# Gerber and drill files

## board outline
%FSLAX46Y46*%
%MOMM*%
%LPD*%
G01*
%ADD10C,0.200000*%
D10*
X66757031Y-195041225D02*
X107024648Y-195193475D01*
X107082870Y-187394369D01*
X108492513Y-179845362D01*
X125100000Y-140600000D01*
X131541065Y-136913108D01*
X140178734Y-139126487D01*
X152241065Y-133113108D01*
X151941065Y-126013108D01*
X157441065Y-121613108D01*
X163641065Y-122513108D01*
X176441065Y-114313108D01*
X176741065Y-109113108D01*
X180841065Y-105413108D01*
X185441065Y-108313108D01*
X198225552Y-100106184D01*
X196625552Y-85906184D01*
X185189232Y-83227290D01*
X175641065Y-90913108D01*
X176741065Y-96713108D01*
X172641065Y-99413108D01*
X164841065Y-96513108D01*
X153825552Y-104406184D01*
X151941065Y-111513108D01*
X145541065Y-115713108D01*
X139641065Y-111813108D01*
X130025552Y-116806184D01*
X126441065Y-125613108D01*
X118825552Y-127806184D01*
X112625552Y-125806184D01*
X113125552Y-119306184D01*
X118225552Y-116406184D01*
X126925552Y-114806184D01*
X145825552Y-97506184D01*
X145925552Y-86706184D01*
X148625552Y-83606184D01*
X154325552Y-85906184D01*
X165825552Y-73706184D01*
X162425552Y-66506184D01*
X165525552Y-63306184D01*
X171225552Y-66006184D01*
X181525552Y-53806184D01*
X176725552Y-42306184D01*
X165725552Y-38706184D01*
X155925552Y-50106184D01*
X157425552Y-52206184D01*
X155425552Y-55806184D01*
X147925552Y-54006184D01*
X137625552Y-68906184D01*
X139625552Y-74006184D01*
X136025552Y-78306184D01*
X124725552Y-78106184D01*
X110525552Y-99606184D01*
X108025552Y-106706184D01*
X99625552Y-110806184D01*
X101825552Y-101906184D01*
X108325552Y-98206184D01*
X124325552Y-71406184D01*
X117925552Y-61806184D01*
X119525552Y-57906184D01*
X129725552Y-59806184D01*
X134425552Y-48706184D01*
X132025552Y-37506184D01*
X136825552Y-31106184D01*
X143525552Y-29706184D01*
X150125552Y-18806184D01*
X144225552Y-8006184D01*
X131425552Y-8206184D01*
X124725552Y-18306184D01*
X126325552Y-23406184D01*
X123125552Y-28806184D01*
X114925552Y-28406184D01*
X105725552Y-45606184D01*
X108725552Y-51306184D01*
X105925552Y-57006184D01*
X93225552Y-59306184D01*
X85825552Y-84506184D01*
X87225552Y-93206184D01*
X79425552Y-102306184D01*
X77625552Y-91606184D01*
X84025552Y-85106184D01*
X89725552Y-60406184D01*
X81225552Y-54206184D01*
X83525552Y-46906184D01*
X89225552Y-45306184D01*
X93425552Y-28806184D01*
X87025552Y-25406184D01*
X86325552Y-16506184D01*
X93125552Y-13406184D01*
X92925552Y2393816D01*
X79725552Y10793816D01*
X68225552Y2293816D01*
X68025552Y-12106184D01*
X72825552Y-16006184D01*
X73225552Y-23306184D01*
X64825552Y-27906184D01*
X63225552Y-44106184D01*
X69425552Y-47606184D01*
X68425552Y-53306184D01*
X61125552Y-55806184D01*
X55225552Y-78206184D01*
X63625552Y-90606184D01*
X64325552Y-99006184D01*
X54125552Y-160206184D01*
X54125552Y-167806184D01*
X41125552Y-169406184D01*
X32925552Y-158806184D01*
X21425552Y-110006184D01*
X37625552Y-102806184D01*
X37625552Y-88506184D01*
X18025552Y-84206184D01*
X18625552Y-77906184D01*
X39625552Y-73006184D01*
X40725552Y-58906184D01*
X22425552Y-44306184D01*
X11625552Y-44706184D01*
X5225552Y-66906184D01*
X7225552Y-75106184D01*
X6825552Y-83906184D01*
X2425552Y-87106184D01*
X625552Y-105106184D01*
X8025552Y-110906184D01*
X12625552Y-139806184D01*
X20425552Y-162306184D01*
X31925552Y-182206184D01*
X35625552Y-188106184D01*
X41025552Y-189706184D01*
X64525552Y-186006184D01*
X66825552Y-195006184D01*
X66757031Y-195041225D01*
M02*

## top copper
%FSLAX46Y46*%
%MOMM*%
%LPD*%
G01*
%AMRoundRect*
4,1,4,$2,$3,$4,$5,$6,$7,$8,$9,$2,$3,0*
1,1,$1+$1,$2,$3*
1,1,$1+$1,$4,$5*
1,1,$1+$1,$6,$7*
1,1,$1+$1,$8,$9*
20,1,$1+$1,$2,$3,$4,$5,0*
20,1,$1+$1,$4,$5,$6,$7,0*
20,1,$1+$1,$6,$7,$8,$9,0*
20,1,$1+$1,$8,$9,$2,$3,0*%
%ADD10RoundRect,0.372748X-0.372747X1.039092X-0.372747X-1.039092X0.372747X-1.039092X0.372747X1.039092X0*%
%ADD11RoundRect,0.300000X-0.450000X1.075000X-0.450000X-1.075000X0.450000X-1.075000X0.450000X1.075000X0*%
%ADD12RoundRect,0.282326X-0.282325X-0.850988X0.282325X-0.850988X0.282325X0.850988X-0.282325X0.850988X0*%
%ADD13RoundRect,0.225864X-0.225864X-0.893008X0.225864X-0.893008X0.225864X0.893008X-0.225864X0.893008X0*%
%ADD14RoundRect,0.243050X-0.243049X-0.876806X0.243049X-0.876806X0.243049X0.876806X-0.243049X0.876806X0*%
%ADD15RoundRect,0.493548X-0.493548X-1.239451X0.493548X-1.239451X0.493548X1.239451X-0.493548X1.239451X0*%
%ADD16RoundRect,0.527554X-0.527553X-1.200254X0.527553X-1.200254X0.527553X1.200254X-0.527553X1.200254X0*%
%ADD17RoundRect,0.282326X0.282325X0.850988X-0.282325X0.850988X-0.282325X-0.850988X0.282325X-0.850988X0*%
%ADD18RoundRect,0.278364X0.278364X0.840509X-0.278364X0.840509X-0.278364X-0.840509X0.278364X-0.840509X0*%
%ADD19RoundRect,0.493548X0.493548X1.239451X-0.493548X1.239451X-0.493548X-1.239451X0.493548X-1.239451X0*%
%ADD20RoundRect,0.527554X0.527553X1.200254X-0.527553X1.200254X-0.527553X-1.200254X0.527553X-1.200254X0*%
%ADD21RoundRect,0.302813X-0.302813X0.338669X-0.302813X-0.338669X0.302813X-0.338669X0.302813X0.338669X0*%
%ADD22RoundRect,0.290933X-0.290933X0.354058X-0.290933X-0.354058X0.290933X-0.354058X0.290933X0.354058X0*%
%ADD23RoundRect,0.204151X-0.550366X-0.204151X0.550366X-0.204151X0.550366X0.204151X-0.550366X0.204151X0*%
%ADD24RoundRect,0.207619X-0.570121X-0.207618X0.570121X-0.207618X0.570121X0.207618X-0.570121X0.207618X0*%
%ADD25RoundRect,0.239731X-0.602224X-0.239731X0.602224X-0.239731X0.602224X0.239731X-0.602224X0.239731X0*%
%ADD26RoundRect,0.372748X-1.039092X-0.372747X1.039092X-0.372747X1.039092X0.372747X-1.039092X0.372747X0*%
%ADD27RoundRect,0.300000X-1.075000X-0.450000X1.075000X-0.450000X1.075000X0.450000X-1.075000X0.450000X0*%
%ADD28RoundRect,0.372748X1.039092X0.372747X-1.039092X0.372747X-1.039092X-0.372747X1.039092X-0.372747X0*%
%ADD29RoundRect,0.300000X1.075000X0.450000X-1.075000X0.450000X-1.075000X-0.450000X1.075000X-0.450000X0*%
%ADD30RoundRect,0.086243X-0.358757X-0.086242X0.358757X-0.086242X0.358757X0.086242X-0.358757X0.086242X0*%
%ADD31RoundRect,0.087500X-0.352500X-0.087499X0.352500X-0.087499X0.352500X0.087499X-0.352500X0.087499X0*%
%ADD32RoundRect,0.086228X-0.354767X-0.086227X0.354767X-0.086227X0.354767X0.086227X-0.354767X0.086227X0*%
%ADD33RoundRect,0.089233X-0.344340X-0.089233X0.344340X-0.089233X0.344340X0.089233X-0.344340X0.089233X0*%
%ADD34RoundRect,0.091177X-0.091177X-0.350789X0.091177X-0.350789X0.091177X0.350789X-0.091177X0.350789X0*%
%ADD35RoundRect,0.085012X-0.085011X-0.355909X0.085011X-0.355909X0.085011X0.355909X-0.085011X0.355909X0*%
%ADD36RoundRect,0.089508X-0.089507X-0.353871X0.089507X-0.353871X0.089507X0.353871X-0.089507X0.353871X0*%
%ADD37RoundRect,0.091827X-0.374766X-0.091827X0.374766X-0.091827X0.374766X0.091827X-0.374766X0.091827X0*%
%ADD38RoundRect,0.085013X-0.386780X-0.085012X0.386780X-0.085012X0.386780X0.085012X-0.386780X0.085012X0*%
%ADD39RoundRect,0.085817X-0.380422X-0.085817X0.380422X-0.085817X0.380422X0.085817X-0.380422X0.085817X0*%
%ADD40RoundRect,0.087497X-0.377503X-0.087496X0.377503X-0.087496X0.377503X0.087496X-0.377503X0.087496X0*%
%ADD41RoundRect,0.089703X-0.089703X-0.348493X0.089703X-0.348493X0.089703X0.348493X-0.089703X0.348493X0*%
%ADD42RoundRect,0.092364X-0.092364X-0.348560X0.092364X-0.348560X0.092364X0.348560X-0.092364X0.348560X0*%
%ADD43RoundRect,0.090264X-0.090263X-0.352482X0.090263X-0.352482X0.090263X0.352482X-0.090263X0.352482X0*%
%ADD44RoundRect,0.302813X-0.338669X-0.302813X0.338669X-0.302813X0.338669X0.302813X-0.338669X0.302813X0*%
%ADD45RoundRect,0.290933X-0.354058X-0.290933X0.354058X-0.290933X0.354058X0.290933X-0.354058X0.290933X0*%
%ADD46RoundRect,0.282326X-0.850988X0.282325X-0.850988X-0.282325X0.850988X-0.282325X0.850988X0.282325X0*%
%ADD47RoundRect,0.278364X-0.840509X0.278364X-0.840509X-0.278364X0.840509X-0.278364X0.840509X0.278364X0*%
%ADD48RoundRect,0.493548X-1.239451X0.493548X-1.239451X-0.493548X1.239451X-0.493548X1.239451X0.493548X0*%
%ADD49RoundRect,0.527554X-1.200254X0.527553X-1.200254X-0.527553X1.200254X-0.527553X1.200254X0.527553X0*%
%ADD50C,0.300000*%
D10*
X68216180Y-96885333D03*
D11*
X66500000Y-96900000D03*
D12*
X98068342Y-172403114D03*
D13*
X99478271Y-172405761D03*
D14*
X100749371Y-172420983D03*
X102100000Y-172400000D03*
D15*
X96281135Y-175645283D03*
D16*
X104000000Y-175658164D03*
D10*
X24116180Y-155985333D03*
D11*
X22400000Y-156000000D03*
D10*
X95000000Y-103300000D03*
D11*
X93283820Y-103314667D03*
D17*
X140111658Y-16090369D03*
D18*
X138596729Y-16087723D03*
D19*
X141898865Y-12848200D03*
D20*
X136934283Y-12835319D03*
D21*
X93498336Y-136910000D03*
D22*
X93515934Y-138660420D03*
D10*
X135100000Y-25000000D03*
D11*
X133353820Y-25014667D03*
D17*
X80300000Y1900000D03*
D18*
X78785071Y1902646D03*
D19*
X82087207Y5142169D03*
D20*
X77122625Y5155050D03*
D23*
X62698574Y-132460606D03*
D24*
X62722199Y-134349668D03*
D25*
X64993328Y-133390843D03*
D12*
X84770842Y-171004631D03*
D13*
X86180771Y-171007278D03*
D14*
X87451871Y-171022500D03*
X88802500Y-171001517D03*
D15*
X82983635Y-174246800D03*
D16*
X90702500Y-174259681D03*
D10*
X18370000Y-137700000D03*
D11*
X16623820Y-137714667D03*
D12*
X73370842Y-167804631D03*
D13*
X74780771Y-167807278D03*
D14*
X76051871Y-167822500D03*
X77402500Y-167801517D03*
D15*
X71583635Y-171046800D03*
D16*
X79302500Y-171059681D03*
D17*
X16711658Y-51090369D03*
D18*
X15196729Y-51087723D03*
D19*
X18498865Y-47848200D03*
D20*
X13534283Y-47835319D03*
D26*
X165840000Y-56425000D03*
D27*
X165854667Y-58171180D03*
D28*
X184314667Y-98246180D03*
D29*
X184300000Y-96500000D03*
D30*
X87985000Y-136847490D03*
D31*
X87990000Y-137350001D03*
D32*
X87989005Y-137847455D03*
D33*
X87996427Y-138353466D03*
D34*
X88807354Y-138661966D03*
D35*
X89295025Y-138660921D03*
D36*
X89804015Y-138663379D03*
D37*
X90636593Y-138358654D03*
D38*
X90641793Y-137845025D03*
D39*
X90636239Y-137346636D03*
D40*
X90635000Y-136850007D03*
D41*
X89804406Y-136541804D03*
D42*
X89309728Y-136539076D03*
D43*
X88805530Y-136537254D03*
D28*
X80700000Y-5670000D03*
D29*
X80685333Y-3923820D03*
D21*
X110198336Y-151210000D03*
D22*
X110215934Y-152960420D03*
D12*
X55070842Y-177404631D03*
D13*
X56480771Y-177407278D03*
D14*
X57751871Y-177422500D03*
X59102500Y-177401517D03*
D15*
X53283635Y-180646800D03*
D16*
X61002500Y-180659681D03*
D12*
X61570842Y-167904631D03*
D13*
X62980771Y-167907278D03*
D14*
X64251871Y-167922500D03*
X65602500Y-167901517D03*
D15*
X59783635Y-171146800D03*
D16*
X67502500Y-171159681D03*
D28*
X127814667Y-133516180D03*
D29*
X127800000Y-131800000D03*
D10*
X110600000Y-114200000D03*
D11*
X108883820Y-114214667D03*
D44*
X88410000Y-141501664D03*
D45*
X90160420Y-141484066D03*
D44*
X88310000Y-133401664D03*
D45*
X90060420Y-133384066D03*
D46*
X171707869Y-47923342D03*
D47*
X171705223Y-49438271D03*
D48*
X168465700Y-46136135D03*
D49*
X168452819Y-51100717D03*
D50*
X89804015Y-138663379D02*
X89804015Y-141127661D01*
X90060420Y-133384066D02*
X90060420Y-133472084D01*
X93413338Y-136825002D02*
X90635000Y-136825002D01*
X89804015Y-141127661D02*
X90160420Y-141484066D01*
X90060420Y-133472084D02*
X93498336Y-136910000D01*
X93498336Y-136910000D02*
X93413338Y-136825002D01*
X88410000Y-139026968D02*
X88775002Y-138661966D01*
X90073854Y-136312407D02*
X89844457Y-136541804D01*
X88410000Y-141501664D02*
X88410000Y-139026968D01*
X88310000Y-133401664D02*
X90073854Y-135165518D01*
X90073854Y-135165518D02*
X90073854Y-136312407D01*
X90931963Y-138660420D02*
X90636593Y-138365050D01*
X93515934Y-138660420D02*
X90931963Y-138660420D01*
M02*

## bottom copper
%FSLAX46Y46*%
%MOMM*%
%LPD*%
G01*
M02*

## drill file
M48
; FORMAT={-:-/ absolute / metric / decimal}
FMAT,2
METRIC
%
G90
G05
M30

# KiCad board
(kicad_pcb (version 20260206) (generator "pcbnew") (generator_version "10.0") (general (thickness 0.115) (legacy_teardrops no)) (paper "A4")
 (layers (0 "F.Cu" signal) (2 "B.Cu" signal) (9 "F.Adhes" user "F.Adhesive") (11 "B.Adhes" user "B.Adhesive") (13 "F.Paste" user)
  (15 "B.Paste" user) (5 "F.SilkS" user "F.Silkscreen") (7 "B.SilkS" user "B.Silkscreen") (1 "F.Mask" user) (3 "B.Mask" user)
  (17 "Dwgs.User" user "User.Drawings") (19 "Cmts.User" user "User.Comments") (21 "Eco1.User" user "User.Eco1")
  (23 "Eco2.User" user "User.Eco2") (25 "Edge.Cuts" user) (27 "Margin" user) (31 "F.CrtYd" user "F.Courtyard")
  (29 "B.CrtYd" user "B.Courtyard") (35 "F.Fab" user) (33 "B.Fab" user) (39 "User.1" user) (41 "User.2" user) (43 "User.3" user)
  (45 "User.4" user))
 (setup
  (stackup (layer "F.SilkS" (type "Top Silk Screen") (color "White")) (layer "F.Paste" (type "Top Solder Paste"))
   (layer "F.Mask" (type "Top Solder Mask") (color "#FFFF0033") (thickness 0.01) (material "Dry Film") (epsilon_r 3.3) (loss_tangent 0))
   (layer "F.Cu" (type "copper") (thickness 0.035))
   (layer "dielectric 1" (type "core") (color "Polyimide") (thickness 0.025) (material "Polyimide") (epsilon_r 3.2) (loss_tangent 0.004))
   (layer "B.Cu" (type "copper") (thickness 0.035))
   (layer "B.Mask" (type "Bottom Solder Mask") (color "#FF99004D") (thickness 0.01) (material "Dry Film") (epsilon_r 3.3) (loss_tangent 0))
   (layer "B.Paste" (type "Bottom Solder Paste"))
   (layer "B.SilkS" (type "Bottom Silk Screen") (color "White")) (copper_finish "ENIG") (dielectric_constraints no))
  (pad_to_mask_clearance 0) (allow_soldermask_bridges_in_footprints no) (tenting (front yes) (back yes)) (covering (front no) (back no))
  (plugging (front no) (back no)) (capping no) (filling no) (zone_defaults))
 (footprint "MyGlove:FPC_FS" (layer "F.Cu") (at 67.37618 96.885333)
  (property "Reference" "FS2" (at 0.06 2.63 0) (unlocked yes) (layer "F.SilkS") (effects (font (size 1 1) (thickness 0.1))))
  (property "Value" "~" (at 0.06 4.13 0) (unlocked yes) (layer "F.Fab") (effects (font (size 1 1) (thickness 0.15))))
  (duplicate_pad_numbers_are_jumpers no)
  (pad "" smd roundrect (at -0.75 0.01 270) (size 2 1) (layers "F.Mask" "F.Paste") (roundrect_rratio 0.2)
   (teardrops (best_length_ratio 0.5) (max_length 1) (best_width_ratio 1) (max_width 2) (curved_edges yes) (filter_ratio 0.9) (enabled yes)
    (allow_two_segments yes) (prefer_zone_connections yes)))
  (pad "" smd roundrect (at 0.75 0.01 270) (size 2 1) (layers "F.Mask" "F.Paste") (roundrect_rratio 0.2)
   (teardrops (best_length_ratio 0.5) (max_length 1) (best_width_ratio 1) (max_width 2) (curved_edges yes) (filter_ratio 0.9) (enabled yes)
    (allow_two_segments yes) (prefer_zone_connections yes)))
  (pad "1" smd roundrect (at 0.84 0 270) (size 2.82368 1.49099) (layers "F.Cu") (roundrect_rratio 0.25) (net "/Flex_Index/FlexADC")
   (teardrops (best_length_ratio 0.5) (max_length 1) (best_width_ratio 1) (max_width 2) (curved_edges yes) (filter_ratio 0.9) (enabled yes)
    (allow_two_segments yes) (prefer_zone_connections yes))
   (padstack (mode custom) (layer "B.Cu" (shape roundrect) (size 2.177876 1.183907) (roundrect_rratio 0.25) (zone_connect -1))))
  (pad "2" smd roundrect (at -0.87618 0.014667 270) (size 2.75 1.5) (layers "F.Cu") (roundrect_rratio 0.2) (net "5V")
   (teardrops (best_length_ratio 0.5) (max_length 1) (best_width_ratio 1) (max_width 2) (curved_edges yes) (filter_ratio 0.9) (enabled yes)
    (allow_two_segments yes) (prefer_zone_connections yes))))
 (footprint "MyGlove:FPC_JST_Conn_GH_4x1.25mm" (layer "F.Cu") (at 95.28 177.970983)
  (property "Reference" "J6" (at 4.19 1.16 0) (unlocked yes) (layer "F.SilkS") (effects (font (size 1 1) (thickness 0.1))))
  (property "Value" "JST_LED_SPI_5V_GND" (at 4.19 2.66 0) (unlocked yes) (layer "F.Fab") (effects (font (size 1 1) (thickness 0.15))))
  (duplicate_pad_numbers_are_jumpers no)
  (pad "" smd roundrect (at 1.065 -2.46) (size 1 2.7) (layers "F.Mask" "F.Paste") (roundrect_rratio 0.25))
  (pad "" smd roundrect (at 2.915 -5.66) (size 0.6 1.7) (layers "F.Mask" "F.Paste") (roundrect_rratio 0.25))
  (pad "" smd roundrect (at 4.165 -5.66) (size 0.6 1.7) (layers "F.Mask" "F.Paste") (roundrect_rratio 0.25))
  (pad "" smd roundrect (at 5.48 -5.61) (size 0.6 1.7) (layers "F.Mask" "F.Paste") (roundrect_rratio 0.25))
  (pad "" smd roundrect (at 6.74 -5.650983) (size 0.6 1.7) (layers "F.Mask" "F.Paste") (roundrect_rratio 0.25))
  (pad "" smd roundrect (at 8.56 -2.46) (size 1 2.7) (layers "F.Mask" "F.Paste") (roundrect_rratio 0.25))
  (pad "1" smd roundrect (at 2.788342 -5.567869) (size 1.129302 2.266628) (layers "F.Cu") (roundrect_rratio 0.25) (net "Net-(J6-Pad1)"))
  (pad "2" smd roundrect (at 4.198271 -5.565222) (size 0.903457 2.237745) (layers "F.Cu") (roundrect_rratio 0.25) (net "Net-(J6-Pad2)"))
  (pad "3" smd roundrect (at 5.469371 -5.55) (size 0.972199 2.239712) (layers "F.Cu") (roundrect_rratio 0.25) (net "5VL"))
  (pad "4" smd roundrect (at 6.82 -5.570983) (size 0.972199 2.239712) (layers "F.Cu") (roundrect_rratio 0.25) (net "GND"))
  (pad "MP" smd roundrect (at 1.001135 -2.3257) (size 1.974193 3.465998) (layers "F.Cu") (roundrect_rratio 0.25))
  (pad "MP" smd roundrect (at 8.72 -2.312819) (size 2.110214 3.455616) (layers "F.Cu") (roundrect_rratio 0.25)))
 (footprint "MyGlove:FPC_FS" (layer "F.Cu") (at 23.27618 155.985333)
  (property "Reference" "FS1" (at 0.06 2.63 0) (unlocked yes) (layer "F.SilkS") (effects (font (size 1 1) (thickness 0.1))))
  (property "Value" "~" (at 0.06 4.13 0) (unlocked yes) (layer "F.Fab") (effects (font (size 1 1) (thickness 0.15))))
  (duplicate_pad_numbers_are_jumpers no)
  (pad "" smd roundrect (at -0.75 0.01 270) (size 2 1) (layers "F.Mask" "F.Paste") (roundrect_rratio 0.2)
   (teardrops (best_length_ratio 0.5) (max_length 1) (best_width_ratio 1) (max_width 2) (curved_edges yes) (filter_ratio 0.9) (enabled yes)
    (allow_two_segments yes) (prefer_zone_connections yes)))
  (pad "" smd roundrect (at 0.75 0.01 270) (size 2 1) (layers "F.Mask" "F.Paste") (roundrect_rratio 0.2)
   (teardrops (best_length_ratio 0.5) (max_length 1) (best_width_ratio 1) (max_width 2) (curved_edges yes) (filter_ratio 0.9) (enabled yes)
    (allow_two_segments yes) (prefer_zone_connections yes)))
  (pad "1" smd roundrect (at 0.84 0 270) (size 2.82368 1.49099) (layers "F.Cu") (roundrect_rratio 0.25) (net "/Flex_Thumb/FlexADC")
   (teardrops (best_length_ratio 0.5) (max_length 1) (best_width_ratio 1) (max_width 2) (curved_edges yes) (filter_ratio 0.9) (enabled yes)
    (allow_two_segments yes) (prefer_zone_connections yes))
   (padstack (mode custom) (layer "B.Cu" (shape roundrect) (size 2.177876 1.183907) (roundrect_rratio 0.25) (zone_connect -1))))
  (pad "2" smd roundrect (at -0.87618 0.014667 270) (size 2.75 1.5) (layers "F.Cu") (roundrect_rratio 0.2) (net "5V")
   (teardrops (best_length_ratio 0.5) (max_length 1) (best_width_ratio 1) (max_width 2) (curved_edges yes) (filter_ratio 0.9) (enabled yes)
    (allow_two_segments yes) (prefer_zone_connections yes))))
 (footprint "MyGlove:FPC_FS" (layer "F.Cu") (at 94.16 103.3)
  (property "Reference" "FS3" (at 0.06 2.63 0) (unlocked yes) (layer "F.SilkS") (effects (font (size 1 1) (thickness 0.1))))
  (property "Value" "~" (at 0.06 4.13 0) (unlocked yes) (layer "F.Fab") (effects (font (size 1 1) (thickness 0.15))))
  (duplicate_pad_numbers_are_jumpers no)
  (pad "" smd roundrect (at -0.75 0.01 270) (size 2 1) (layers "F.Mask" "F.Paste") (roundrect_rratio 0.2)
   (teardrops (best_length_ratio 0.5) (max_length 1) (best_width_ratio 1) (max_width 2) (curved_edges yes) (filter_ratio 0.9) (enabled yes)
    (allow_two_segments yes) (prefer_zone_connections yes)))
  (pad "" smd roundrect (at 0.75 0.01 270) (size 2 1) (layers "F.Mask" "F.Paste") (roundrect_rratio 0.2)
   (teardrops (best_length_ratio 0.5) (max_length 1) (best_width_ratio 1) (max_width 2) (curved_edges yes) (filter_ratio 0.9) (enabled yes)
    (allow_two_segments yes) (prefer_zone_connections yes)))
  (pad "1" smd roundrect (at 0.84 0 270) (size 2.82368 1.49099) (layers "F.Cu") (roundrect_rratio 0.25) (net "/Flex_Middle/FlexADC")
   (teardrops (best_length_ratio 0.5) (max_length 1) (best_width_ratio 1) (max_width 2) (curved_edges yes) (filter_ratio 0.9) (enabled yes)
    (allow_two_segments yes) (prefer_zone_connections yes))
   (padstack (mode custom) (layer "B.Cu" (shape roundrect) (size 2.177876 1.183907) (roundrect_rratio 0.25) (zone_connect -1))))
  (pad "2" smd roundrect (at -0.87618 0.014667 270) (size 2.75 1.5) (layers "F.Cu") (roundrect_rratio 0.2) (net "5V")
   (teardrops (best_length_ratio 0.5) (max_length 1) (best_width_ratio 1) (max_width 2) (curved_edges yes) (filter_ratio 0.9) (enabled yes)
    (allow_two_segments yes) (prefer_zone_connections yes))))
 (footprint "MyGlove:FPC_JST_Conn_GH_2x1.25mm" (layer "F.Cu") (at 142.9 10.5225 180)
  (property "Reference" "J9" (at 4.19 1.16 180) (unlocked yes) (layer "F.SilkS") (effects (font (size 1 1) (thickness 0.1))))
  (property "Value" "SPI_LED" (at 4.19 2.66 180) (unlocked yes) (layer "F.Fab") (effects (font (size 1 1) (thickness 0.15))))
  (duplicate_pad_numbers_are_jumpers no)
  (pad "" smd roundrect (at 1.065 -2.46 180) (size 1 2.7) (layers "F.Mask" "F.Paste") (roundrect_rratio 0.25))
  (pad "" smd roundrect (at 2.915 -5.66 180) (size 0.6 1.7) (layers "F.Mask" "F.Paste") (roundrect_rratio 0.25))
  (pad "" smd roundrect (at 4.165 -5.66 180) (size 0.6 1.7) (layers "F.Mask" "F.Paste") (roundrect_rratio 0.25))
  (pad "" smd roundrect (at 6.015 -2.46 180) (size 1 2.7) (layers "F.Mask" "F.Paste") (roundrect_rratio 0.25))
  (pad "1" smd roundrect (at 2.788342 -5.567869 180) (size 1.129302 2.266628) (layers "F.Cu") (roundrect_rratio 0.25) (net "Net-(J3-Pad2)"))
  (pad "2" smd roundrect (at 4.303271 -5.565223 180) (size 1.113457 2.237746) (layers "F.Cu") (roundrect_rratio 0.25) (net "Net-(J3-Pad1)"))
  (pad "MP" smd roundrect (at 1.001135 -2.3257 180) (size 1.974193 3.465998) (layers "F.Cu") (roundrect_rratio 0.25))
  (pad "MP" smd roundrect (at 5.965717 -2.312819 180) (size 2.110214 3.455616) (layers "F.Cu") (roundrect_rratio 0.25)))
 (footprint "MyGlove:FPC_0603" (layer "F.Cu") (at 93.5 137.8 -90)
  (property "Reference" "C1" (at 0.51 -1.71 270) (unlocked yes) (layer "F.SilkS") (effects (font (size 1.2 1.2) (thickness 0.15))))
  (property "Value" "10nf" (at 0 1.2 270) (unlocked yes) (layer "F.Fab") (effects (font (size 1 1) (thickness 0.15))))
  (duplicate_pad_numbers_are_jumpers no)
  (pad "" smd roundrect (at -0.87 0.005971 270) (size 1.00047 0.948058) (layers "F.Mask" "F.Paste") (roundrect_rratio 0.2))
  (pad "" smd roundrect (at 0.85 0 270) (size 1.054536 0.970792) (layers "F.Mask" "F.Paste") (roundrect_rratio 0.2))
  (pad "1" smd roundrect (at -0.89 0.001664 270) (size 1.282964 1.211252) (layers "F.Cu") (roundrect_rratio 0.25) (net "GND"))
  (pad "2" smd roundrect (at 0.86042 -0.015934 270) (size 1.289982 1.163733) (layers "F.Cu") (roundrect_rratio 0.25) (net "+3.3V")))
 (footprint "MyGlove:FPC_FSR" (layer "F.Cu") (at 134.23 25)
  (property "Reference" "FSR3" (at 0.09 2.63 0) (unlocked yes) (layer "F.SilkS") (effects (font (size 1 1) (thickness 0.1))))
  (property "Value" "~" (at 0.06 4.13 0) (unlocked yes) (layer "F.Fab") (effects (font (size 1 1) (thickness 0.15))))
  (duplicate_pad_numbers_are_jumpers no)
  (pad "" smd roundrect (at -0.75 0.01 270) (size 2 1) (layers "F.Mask" "F.Paste") (roundrect_rratio 0.2)
   (teardrops (best_length_ratio 0.5) (max_length 1) (best_width_ratio 1) (max_width 2) (curved_edges yes) (filter_ratio 0.9) (enabled yes)
    (allow_two_segments yes) (prefer_zone_connections yes)))
  (pad "" smd roundrect (at 0.78 0.01 270) (size 2 1) (layers "F.Mask" "F.Paste") (roundrect_rratio 0.2)
   (teardrops (best_length_ratio 0.5) (max_length 1) (best_width_ratio 1) (max_width 2) (curved_edges yes) (filter_ratio 0.9) (enabled yes)
    (allow_two_segments yes) (prefer_zone_connections yes)))
  (pad "1" smd roundrect (at 0.87 0 270) (size 2.82368 1.49099) (layers "F.Cu") (roundrect_rratio 0.25) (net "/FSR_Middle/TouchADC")
   (teardrops (best_length_ratio 0.5) (max_length 1) (best_width_ratio 1) (max_width 2) (curved_edges yes) (filter_ratio 0.9) (enabled yes)
    (allow_two_segments yes) (prefer_zone_connections yes))
   (padstack (mode custom) (layer "B.Cu" (shape roundrect) (size 2.177876 1.183907) (roundrect_rratio 0.25) (zone_connect -1))))
  (pad "2" smd roundrect (at -0.87618 0.014667 270) (size 2.75 1.5) (layers "F.Cu") (roundrect_rratio 0.2) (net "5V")
   (teardrops (best_length_ratio 0.5) (max_length 1) (best_width_ratio 1) (max_width 2) (curved_edges yes) (filter_ratio 0.9) (enabled yes)
    (allow_two_segments yes) (prefer_zone_connections yes))))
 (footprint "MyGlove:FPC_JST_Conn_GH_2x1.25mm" (layer "F.Cu") (at 83.088342 -7.467869 180)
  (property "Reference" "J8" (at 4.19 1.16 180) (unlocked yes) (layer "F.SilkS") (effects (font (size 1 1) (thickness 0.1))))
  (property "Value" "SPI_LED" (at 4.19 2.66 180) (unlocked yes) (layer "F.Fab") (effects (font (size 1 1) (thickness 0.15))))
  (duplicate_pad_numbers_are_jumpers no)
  (pad "" smd roundrect (at 1.065 -2.46 180) (size 1 2.7) (layers "F.Mask" "F.Paste") (roundrect_rratio 0.25))
  (pad "" smd roundrect (at 2.915 -5.66 180) (size 0.6 1.7) (layers "F.Mask" "F.Paste") (roundrect_rratio 0.25))
  (pad "" smd roundrect (at 4.165 -5.66 180) (size 0.6 1.7) (layers "F.Mask" "F.Paste") (roundrect_rratio 0.25))
  (pad "" smd roundrect (at 6.015 -2.46 180) (size 1 2.7) (layers "F.Mask" "F.Paste") (roundrect_rratio 0.25))
  (pad "1" smd roundrect (at 2.788342 -5.567869 180) (size 1.129302 2.266628) (layers "F.Cu") (roundrect_rratio 0.25) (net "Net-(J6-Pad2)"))
  (pad "2" smd roundrect (at 4.303271 -5.565223 180) (size 1.113457 2.237746) (layers "F.Cu") (roundrect_rratio 0.25) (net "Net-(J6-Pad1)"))
  (pad "MP" smd roundrect (at 1.001135 -2.3257 180) (size 1.974193 3.465998) (layers "F.Cu") (roundrect_rratio 0.25))
  (pad "MP" smd roundrect (at 5.965717 -2.312819 180) (size 2.110214 3.455616) (layers "F.Cu") (roundrect_rratio 0.25)))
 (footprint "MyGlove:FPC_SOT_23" (layer "F.Cu") (at 63.8425 133.37)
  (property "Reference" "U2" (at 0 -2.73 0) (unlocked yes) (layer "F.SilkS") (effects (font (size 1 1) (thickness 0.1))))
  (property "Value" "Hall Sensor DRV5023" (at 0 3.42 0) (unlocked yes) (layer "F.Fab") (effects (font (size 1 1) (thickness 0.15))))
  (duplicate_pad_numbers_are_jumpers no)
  (pad "" smd roundrect (at -1.1175 -0.92) (size 1.325 0.6) (layers "F.Mask" "F.Paste") (roundrect_rratio 0.25))
  (pad "" smd roundrect (at -1.1175 0.98) (size 1.325 0.6) (layers "F.Mask" "F.Paste") (roundrect_rratio 0.25))
  (pad "" smd roundrect (at 1.1575 0.03) (size 1.325 0.6) (layers "F.Mask" "F.Paste") (roundrect_rratio 0.25))
  (pad "1" smd roundrect (at -1.143926 -0.909394) (size 1.509034 0.816604) (layers "F.Cu") (roundrect_rratio 0.25) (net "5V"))
  (pad "2" smd roundrect (at -1.120301 0.979668) (size 1.555481 0.830475) (layers "F.Cu") (roundrect_rratio 0.25) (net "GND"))
  (pad "3" smd roundrect (at 1.150828 0.020843) (size 1.683911 0.958924) (layers "F.Cu") (roundrect_rratio 0.25)
   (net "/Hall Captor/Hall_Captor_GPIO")))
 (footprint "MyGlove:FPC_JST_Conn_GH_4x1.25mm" (layer "F.Cu") (at 81.9825 176.5725)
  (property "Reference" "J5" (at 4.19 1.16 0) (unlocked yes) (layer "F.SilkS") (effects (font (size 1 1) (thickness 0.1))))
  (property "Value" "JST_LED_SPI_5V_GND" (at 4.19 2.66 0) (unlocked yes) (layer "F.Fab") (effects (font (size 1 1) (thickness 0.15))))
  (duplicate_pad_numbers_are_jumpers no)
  (pad "" smd roundrect (at 1.065 -2.46) (size 1 2.7) (layers "F.Mask" "F.Paste") (roundrect_rratio 0.25))
  (pad "" smd roundrect (at 2.915 -5.66) (size 0.6 1.7) (layers "F.Mask" "F.Paste") (roundrect_rratio 0.25))
  (pad "" smd roundrect (at 4.165 -5.66) (size 0.6 1.7) (layers "F.Mask" "F.Paste") (roundrect_rratio 0.25))
  (pad "" smd roundrect (at 5.48 -5.61) (size 0.6 1.7) (layers "F.Mask" "F.Paste") (roundrect_rratio 0.25))
  (pad "" smd roundrect (at 6.74 -5.650983) (size 0.6 1.7) (layers "F.Mask" "F.Paste") (roundrect_rratio 0.25))
  (pad "" smd roundrect (at 8.56 -2.46) (size 1 2.7) (layers "F.Mask" "F.Paste") (roundrect_rratio 0.25))
  (pad "1" smd roundrect (at 2.788342 -5.567869) (size 1.129302 2.266628) (layers "F.Cu") (roundrect_rratio 0.25) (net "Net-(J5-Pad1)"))
  (pad "2" smd roundrect (at 4.198271 -5.565222) (size 0.903457 2.237745) (layers "F.Cu") (roundrect_rratio 0.25) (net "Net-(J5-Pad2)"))
  (pad "3" smd roundrect (at 5.469371 -5.55) (size 0.972199 2.239712) (layers "F.Cu") (roundrect_rratio 0.25) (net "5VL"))
  (pad "4" smd roundrect (at 6.82 -5.570983) (size 0.972199 2.239712) (layers "F.Cu") (roundrect_rratio 0.25) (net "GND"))
  (pad "MP" smd roundrect (at 1.001135 -2.3257) (size 1.974193 3.465998) (layers "F.Cu") (roundrect_rratio 0.25))
  (pad "MP" smd roundrect (at 8.72 -2.312819) (size 2.110214 3.455616) (layers "F.Cu") (roundrect_rratio 0.25)))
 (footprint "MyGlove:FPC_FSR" (layer "F.Cu") (at 17.5 137.7)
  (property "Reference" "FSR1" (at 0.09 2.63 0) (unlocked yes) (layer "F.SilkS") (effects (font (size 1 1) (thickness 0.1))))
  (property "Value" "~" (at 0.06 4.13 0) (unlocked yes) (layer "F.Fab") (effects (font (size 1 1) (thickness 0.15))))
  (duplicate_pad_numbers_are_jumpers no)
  (pad "" smd roundrect (at -0.75 0.01 270) (size 2 1) (layers "F.Mask" "F.Paste") (roundrect_rratio 0.2)
   (teardrops (best_length_ratio 0.5) (max_length 1) (best_width_ratio 1) (max_width 2) (curved_edges yes) (filter_ratio 0.9) (enabled yes)
    (allow_two_segments yes) (prefer_zone_connections yes)))
  (pad "" smd roundrect (at 0.78 0.01 270) (size 2 1) (layers "F.Mask" "F.Paste") (roundrect_rratio 0.2)
   (teardrops (best_length_ratio 0.5) (max_length 1) (best_width_ratio 1) (max_width 2) (curved_edges yes) (filter_ratio 0.9) (enabled yes)
    (allow_two_segments yes) (prefer_zone_connections yes)))
  (pad "1" smd roundrect (at 0.87 0 270) (size 2.82368 1.49099) (layers "F.Cu") (roundrect_rratio 0.25) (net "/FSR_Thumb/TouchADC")
   (teardrops (best_length_ratio 0.5) (max_length 1) (best_width_ratio 1) (max_width 2) (curved_edges yes) (filter_ratio 0.9) (enabled yes)
    (allow_two_segments yes) (prefer_zone_connections yes))
   (padstack (mode custom) (layer "B.Cu" (shape roundrect) (size 2.177876 1.183907) (roundrect_rratio 0.25) (zone_connect -1))))
  (pad "2" smd roundrect (at -0.87618 0.014667 270) (size 2.75 1.5) (layers "F.Cu") (roundrect_rratio 0.2) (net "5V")
   (teardrops (best_length_ratio 0.5) (max_length 1) (best_width_ratio 1) (max_width 2) (curved_edges yes) (filter_ratio 0.9) (enabled yes)
    (allow_two_segments yes) (prefer_zone_connections yes))))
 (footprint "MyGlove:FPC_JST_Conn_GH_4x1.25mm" (layer "F.Cu") (at 70.5825 173.3725)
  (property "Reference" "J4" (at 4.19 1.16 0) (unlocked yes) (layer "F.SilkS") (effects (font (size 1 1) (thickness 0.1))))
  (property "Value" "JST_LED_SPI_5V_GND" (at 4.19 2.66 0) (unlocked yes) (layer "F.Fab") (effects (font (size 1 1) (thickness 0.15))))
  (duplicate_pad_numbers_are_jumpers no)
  (pad "" smd roundrect (at 1.065 -2.46) (size 1 2.7) (layers "F.Mask" "F.Paste") (roundrect_rratio 0.25))
  (pad "" smd roundrect (at 2.915 -5.66) (size 0.6 1.7) (layers "F.Mask" "F.Paste") (roundrect_rratio 0.25))
  (pad "" smd roundrect (at 4.165 -5.66) (size 0.6 1.7) (layers "F.Mask" "F.Paste") (roundrect_rratio 0.25))
  (pad "" smd roundrect (at 5.48 -5.61) (size 0.6 1.7) (layers "F.Mask" "F.Paste") (roundrect_rratio 0.25))
  (pad "" smd roundrect (at 6.74 -5.650983) (size 0.6 1.7) (layers "F.Mask" "F.Paste") (roundrect_rratio 0.25))
  (pad "" smd roundrect (at 8.56 -2.46) (size 1 2.7) (layers "F.Mask" "F.Paste") (roundrect_rratio 0.25))
  (pad "1" smd roundrect (at 2.788342 -5.567869) (size 1.129302 2.266628) (layers "F.Cu") (roundrect_rratio 0.25)
   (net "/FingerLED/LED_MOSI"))
  (pad "2" smd roundrect (at 4.198271 -5.565222) (size 0.903457 2.237745) (layers "F.Cu") (roundrect_rratio 0.25) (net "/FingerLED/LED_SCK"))
  (pad "3" smd roundrect (at 5.469371 -5.55) (size 0.972199 2.239712) (layers "F.Cu") (roundrect_rratio 0.25) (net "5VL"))
  (pad "4" smd roundrect (at 6.82 -5.570983) (size 0.972199 2.239712) (layers "F.Cu") (roundrect_rratio 0.25) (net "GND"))
  (pad "MP" smd roundrect (at 1.001135 -2.3257) (size 1.974193 3.465998) (layers "F.Cu") (roundrect_rratio 0.25))
  (pad "MP" smd roundrect (at 8.72 -2.312819) (size 2.110214 3.455616) (layers "F.Cu") (roundrect_rratio 0.25)))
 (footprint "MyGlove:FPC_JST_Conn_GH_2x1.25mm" (layer "F.Cu") (at 19.5 45.5225 180)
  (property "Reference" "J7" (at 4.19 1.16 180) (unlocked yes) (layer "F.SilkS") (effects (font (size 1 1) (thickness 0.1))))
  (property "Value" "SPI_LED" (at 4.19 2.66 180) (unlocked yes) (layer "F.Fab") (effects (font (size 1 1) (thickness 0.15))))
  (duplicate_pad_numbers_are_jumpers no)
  (pad "" smd roundrect (at 1.065 -2.46 180) (size 1 2.7) (layers "F.Mask" "F.Paste") (roundrect_rratio 0.25))
  (pad "" smd roundrect (at 2.915 -5.66 180) (size 0.6 1.7) (layers "F.Mask" "F.Paste") (roundrect_rratio 0.25))
  (pad "" smd roundrect (at 4.165 -5.66 180) (size 0.6 1.7) (layers "F.Mask" "F.Paste") (roundrect_rratio 0.25))
  (pad "" smd roundrect (at 6.015 -2.46 180) (size 1 2.7) (layers "F.Mask" "F.Paste") (roundrect_rratio 0.25))
  (pad "1" smd roundrect (at 2.788342 -5.567869 180) (size 1.129302 2.266628) (layers "F.Cu") (roundrect_rratio 0.25) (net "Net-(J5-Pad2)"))
  (pad "2" smd roundrect (at 4.303271 -5.565223 180) (size 1.113457 2.237746) (layers "F.Cu") (roundrect_rratio 0.25) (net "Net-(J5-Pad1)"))
  (pad "MP" smd roundrect (at 1.001135 -2.3257 180) (size 1.974193 3.465998) (layers "F.Cu") (roundrect_rratio 0.25))
  (pad "MP" smd roundrect (at 5.965717 -2.312819 180) (size 2.110214 3.455616) (layers "F.Cu") (roundrect_rratio 0.25)))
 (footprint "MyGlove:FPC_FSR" (layer "F.Cu") (at 165.84 57.295 90)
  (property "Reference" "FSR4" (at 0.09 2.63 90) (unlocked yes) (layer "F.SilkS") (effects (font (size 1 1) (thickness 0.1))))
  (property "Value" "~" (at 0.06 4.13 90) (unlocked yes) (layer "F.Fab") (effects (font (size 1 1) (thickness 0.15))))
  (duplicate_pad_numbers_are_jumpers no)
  (pad "" smd roundrect (at -0.75 0.01) (size 2 1) (layers "F.Mask" "F.Paste") (roundrect_rratio 0.2)
   (teardrops (best_length_ratio 0.5) (max_length 1) (best_width_ratio 1) (max_width 2) (curved_edges yes) (filter_ratio 0.9) (enabled yes)
    (allow_two_segments yes) (prefer_zone_connections yes)))
  (pad "" smd roundrect (at 0.78 0.01) (size 2 1) (layers "F.Mask" "F.Paste") (roundrect_rratio 0.2)
   (teardrops (best_length_ratio 0.5) (max_length 1) (best_width_ratio 1) (max_width 2) (curved_edges yes) (filter_ratio 0.9) (enabled yes)
    (allow_two_segments yes) (prefer_zone_connections yes)))
  (pad "1" smd roundrect (at 0.87 0) (size 2.82368 1.49099) (layers "F.Cu") (roundrect_rratio 0.25) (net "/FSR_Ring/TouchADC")
   (teardrops (best_length_ratio 0.5) (max_length 1) (best_width_ratio 1) (max_width 2) (curved_edges yes) (filter_ratio 0.9) (enabled yes)
    (allow_two_segments yes) (prefer_zone_connections yes))
   (padstack (mode custom) (layer "B.Cu" (shape roundrect) (size 2.177876 1.183907) (roundrect_rratio 0.25) (zone_connect -1))))
  (pad "2" smd roundrect (at -0.87618 0.014667) (size 2.75 1.5) (layers "F.Cu") (roundrect_rratio 0.2) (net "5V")
   (teardrops (best_length_ratio 0.5) (max_length 1) (best_width_ratio 1) (max_width 2) (curved_edges yes) (filter_ratio 0.9) (enabled yes)
    (allow_two_segments yes) (prefer_zone_connections yes))))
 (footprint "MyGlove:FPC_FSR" (layer "F.Cu") (at 184.314667 97.37618 -90)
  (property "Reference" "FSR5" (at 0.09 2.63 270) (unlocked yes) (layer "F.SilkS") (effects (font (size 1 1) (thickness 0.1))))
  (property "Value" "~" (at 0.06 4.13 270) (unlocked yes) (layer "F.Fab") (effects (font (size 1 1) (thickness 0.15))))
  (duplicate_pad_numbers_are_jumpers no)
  (pad "" smd roundrect (at -0.75 0.01 180) (size 2 1) (layers "F.Mask" "F.Paste") (roundrect_rratio 0.2)
   (teardrops (best_length_ratio 0.5) (max_length 1) (best_width_ratio 1) (max_width 2) (curved_edges yes) (filter_ratio 0.9) (enabled yes)
    (allow_two_segments yes) (prefer_zone_connections yes)))
  (pad "" smd roundrect (at 0.78 0.01 180) (size 2 1) (layers "F.Mask" "F.Paste") (roundrect_rratio 0.2)
   (teardrops (best_length_ratio 0.5) (max_length 1) (best_width_ratio 1) (max_width 2) (curved_edges yes) (filter_ratio 0.9) (enabled yes)
    (allow_two_segments yes) (prefer_zone_connections yes)))
  (pad "1" smd roundrect (at 0.87 0 180) (size 2.82368 1.49099) (layers "F.Cu") (roundrect_rratio 0.25) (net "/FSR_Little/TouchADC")
   (teardrops (best_length_ratio 0.5) (max_length 1) (best_width_ratio 1) (max_width 2) (curved_edges yes) (filter_ratio 0.9) (enabled yes)
    (allow_two_segments yes) (prefer_zone_connections yes))
   (padstack (mode custom) (layer "B.Cu" (shape roundrect) (size 2.177876 1.183907) (roundrect_rratio 0.25) (zone_connect -1))))
  (pad "2" smd roundrect (at -0.87618 0.014667 180) (size 2.75 1.5) (layers "F.Cu") (roundrect_rratio 0.2) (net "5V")
   (teardrops (best_length_ratio 0.5) (max_length 1) (best_width_ratio 1) (max_width 2) (curved_edges yes) (filter_ratio 0.9) (enabled yes)
    (allow_two_segments yes) (prefer_zone_connections yes))))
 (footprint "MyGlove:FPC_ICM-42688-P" (layer "F.Cu") (at 89.3 137.6)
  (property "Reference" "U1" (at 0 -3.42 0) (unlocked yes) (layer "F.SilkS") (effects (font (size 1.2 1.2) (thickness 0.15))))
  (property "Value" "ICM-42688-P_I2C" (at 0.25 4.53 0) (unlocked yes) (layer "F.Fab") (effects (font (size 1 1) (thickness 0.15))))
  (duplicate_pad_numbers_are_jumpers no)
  (pad "1" smd roundrect (at -1.315 -0.75251) (size 0.89 0.344971) (layers "F.Cu" "F.Mask" "F.Paste") (roundrect_rratio 0.25)
   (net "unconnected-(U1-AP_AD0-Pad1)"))
  (pad "2" smd roundrect (at -1.31 -0.249999) (size 0.88 0.349998) (layers "F.Cu" "F.Mask" "F.Paste") (roundrect_rratio 0.25)
   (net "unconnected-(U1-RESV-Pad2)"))
  (pad "3" smd roundrect (at -1.310995 0.247455) (size 0.88199 0.344911) (layers "F.Cu" "F.Mask" "F.Paste") (roundrect_rratio 0.25)
   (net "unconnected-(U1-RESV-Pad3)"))
  (pad "4" smd roundrect (at -1.303573 0.753466) (size 0.867147 0.356932) (layers "F.Cu" "F.Mask" "F.Paste") (roundrect_rratio 0.25)
   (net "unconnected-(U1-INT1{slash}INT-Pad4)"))
  (pad "5" smd roundrect (at -0.492646 1.061966) (size 0.364708 0.883932) (layers "F.Cu" "F.Mask" "F.Paste") (roundrect_rratio 0.25)
   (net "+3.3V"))
  (pad "6" smd roundrect (at -0.004975 1.060921) (size 0.340046 0.881843) (layers "F.Cu" "F.Mask" "F.Paste") (roundrect_rratio 0.25)
   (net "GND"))
  (pad "7" smd roundrect (at 0.504015 1.063379) (size 0.358031 0.886758) (layers "F.Cu" "F.Mask" "F.Paste") (roundrect_rratio 0.25)
   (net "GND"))
  (pad "8" smd roundrect (at 1.336593 0.758654) (size 0.933187 0.367308) (layers "F.Cu" "F.Mask" "F.Paste") (roundrect_rratio 0.25)
   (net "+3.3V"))
  (pad "9" smd roundrect (at 1.341793 0.245025) (size 0.943586 0.34005) (layers "F.Cu" "F.Mask" "F.Paste") (roundrect_rratio 0.25)
   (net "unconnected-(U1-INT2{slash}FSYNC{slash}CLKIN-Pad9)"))
  (pad "10" smd roundrect (at 1.336239 -0.253364) (size 0.932478 0.343268) (layers "F.Cu" "F.Mask" "F.Paste") (roundrect_rratio 0.25)
   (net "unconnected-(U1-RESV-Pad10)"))
  (pad "11" smd roundrect (at 1.335 -0.749993) (size 0.93 0.349986) (layers "F.Cu" "F.Mask" "F.Paste") (roundrect_rratio 0.25) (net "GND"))
  (pad "12" smd roundrect (at 0.504406 -1.058196) (size 0.358813 0.876392) (layers "F.Cu" "F.Mask" "F.Paste") (roundrect_rratio 0.25)
   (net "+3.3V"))
  (pad "13" smd roundrect (at 0.009728 -1.060924) (size 0.369457 0.881848) (layers "F.Cu" "F.Mask" "F.Paste") (roundrect_rratio 0.25)
   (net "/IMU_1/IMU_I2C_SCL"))
  (pad "14" smd roundrect (at -0.49447 -1.062746) (size 0.361054 0.885492) (layers "F.Cu" "F.Mask" "F.Paste") (roundrect_rratio 0.25)
   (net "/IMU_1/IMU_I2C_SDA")))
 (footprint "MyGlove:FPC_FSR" (layer "F.Cu") (at 80.7 4.8 -90)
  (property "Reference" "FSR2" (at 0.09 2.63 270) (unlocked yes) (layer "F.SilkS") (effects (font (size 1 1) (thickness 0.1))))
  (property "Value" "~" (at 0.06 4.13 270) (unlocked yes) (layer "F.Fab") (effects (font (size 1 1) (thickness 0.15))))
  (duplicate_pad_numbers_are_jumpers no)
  (pad "" smd roundrect (at -0.75 0.01 180) (size 2 1) (layers "F.Mask" "F.Paste") (roundrect_rratio 0.2)
   (teardrops (best_length_ratio 0.5) (max_length 1) (best_width_ratio 1) (max_width 2) (curved_edges yes) (filter_ratio 0.9) (enabled yes)
    (allow_two_segments yes) (prefer_zone_connections yes)))
  (pad "" smd roundrect (at 0.78 0.01 180) (size 2 1) (layers "F.Mask" "F.Paste") (roundrect_rratio 0.2)
   (teardrops (best_length_ratio 0.5) (max_length 1) (best_width_ratio 1) (max_width 2) (curved_edges yes) (filter_ratio 0.9) (enabled yes)
    (allow_two_segments yes) (prefer_zone_connections yes)))
  (pad "1" smd roundrect (at 0.87 0 180) (size 2.82368 1.49099) (layers "F.Cu") (roundrect_rratio 0.25) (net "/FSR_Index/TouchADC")
   (teardrops (best_length_ratio 0.5) (max_length 1) (best_width_ratio 1) (max_width 2) (curved_edges yes) (filter_ratio 0.9) (enabled yes)
    (allow_two_segments yes) (prefer_zone_connections yes))
   (padstack (mode custom) (layer "B.Cu" (shape roundrect) (size 2.177876 1.183907) (roundrect_rratio 0.25) (zone_connect -1))))
  (pad "2" smd roundrect (at -0.87618 0.014667 180) (size 2.75 1.5) (layers "F.Cu") (roundrect_rratio 0.2) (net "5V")
   (teardrops (best_length_ratio 0.5) (max_length 1) (best_width_ratio 1) (max_width 2) (curved_edges yes) (filter_ratio 0.9) (enabled yes)
    (allow_two_segments yes) (prefer_zone_connections yes))))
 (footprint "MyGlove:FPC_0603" (layer "F.Cu") (at 110.2 152.1 -90)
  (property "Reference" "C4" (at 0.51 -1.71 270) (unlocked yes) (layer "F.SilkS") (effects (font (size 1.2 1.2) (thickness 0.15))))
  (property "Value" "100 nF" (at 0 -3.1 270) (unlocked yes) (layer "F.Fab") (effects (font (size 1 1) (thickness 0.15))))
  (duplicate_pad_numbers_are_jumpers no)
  (pad "" smd roundrect (at -0.87 0.005971 270) (size 1.00047 0.948058) (layers "F.Mask" "F.Paste") (roundrect_rratio 0.2))
  (pad "" smd roundrect (at 0.85 0 270) (size 1.054536 0.970792) (layers "F.Mask" "F.Paste") (roundrect_rratio 0.2))
  (pad "1" smd roundrect (at -0.89 0.001664 270) (size 1.282964 1.211252) (layers "F.Cu") (roundrect_rratio 0.25) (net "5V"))
  (pad "2" smd roundrect (at 0.86042 -0.015934 270) (size 1.289982 1.163733) (layers "F.Cu") (roundrect_rratio 0.25) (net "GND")))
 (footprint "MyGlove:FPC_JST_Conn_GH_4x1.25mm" (layer "F.Cu") (at 52.2825 182.9725)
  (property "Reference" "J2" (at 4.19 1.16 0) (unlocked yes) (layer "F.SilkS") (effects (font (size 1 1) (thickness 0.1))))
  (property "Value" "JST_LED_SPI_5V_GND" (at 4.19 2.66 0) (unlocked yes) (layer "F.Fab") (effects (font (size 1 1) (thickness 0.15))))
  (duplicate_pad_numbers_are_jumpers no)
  (pad "" smd roundrect (at 1.065 -2.46) (size 1 2.7) (layers "F.Mask" "F.Paste") (roundrect_rratio 0.25))
  (pad "" smd roundrect (at 2.915 -5.66) (size 0.6 1.7) (layers "F.Mask" "F.Paste") (roundrect_rratio 0.25))
  (pad "" smd roundrect (at 4.165 -5.66) (size 0.6 1.7) (layers "F.Mask" "F.Paste") (roundrect_rratio 0.25))
  (pad "" smd roundrect (at 5.48 -5.61) (size 0.6 1.7) (layers "F.Mask" "F.Paste") (roundrect_rratio 0.25))
  (pad "" smd roundrect (at 6.74 -5.650983) (size 0.6 1.7) (layers "F.Mask" "F.Paste") (roundrect_rratio 0.25))
  (pad "" smd roundrect (at 8.56 -2.46) (size 1 2.7) (layers "F.Mask" "F.Paste") (roundrect_rratio 0.25))
  (pad "1" smd roundrect (at 2.788342 -5.567869) (size 1.129302 2.266628) (layers "F.Cu") (roundrect_rratio 0.25) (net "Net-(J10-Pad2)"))
  (pad "2" smd roundrect (at 4.198271 -5.565222) (size 0.903457 2.237745) (layers "F.Cu") (roundrect_rratio 0.25) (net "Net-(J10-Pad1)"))
  (pad "3" smd roundrect (at 5.469371 -5.55) (size 0.972199 2.239712) (layers "F.Cu") (roundrect_rratio 0.25) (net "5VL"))
  (pad "4" smd roundrect (at 6.82 -5.570983) (size 0.972199 2.239712) (layers "F.Cu") (roundrect_rratio 0.25) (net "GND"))
  (pad "MP" smd roundrect (at 1.001135 -2.3257) (size 1.974193 3.465998) (layers "F.Cu") (roundrect_rratio 0.25))
  (pad "MP" smd roundrect (at 8.72 -2.312819) (size 2.110214 3.455616) (layers "F.Cu") (roundrect_rratio 0.25)))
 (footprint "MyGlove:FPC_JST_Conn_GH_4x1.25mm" (layer "F.Cu") (at 58.7825 173.4725)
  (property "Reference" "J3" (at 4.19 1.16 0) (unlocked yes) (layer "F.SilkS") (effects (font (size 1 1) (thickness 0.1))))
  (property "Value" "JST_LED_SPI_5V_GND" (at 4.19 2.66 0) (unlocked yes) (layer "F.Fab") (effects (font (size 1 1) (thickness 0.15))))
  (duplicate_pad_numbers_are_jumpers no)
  (pad "" smd roundrect (at 1.065 -2.46) (size 1 2.7) (layers "F.Mask" "F.Paste") (roundrect_rratio 0.25))
  (pad "" smd roundrect (at 2.915 -5.66) (size 0.6 1.7) (layers "F.Mask" "F.Paste") (roundrect_rratio 0.25))
  (pad "" smd roundrect (at 4.165 -5.66) (size 0.6 1.7) (layers "F.Mask" "F.Paste") (roundrect_rratio 0.25))
  (pad "" smd roundrect (at 5.48 -5.61) (size 0.6 1.7) (layers "F.Mask" "F.Paste") (roundrect_rratio 0.25))
  (pad "" smd roundrect (at 6.74 -5.650983) (size 0.6 1.7) (layers "F.Mask" "F.Paste") (roundrect_rratio 0.25))
  (pad "" smd roundrect (at 8.56 -2.46) (size 1 2.7) (layers "F.Mask" "F.Paste") (roundrect_rratio 0.25))
  (pad "1" smd roundrect (at 2.788342 -5.567869) (size 1.129302 2.266628) (layers "F.Cu") (roundrect_rratio 0.25) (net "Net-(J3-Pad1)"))
  (pad "2" smd roundrect (at 4.198271 -5.565222) (size 0.903457 2.237745) (layers "F.Cu") (roundrect_rratio 0.25) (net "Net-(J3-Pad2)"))
  (pad "3" smd roundrect (at 5.469371 -5.55) (size 0.972199 2.239712) (layers "F.Cu") (roundrect_rratio 0.25) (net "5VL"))
  (pad "4" smd roundrect (at 6.82 -5.570983) (size 0.972199 2.239712) (layers "F.Cu") (roundrect_rratio 0.25) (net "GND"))
  (pad "MP" smd roundrect (at 1.001135 -2.3257) (size 1.974193 3.465998) (layers "F.Cu") (roundrect_rratio 0.25))
  (pad "MP" smd roundrect (at 8.72 -2.312819) (size 2.110214 3.455616) (layers "F.Cu") (roundrect_rratio 0.25)))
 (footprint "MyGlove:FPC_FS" (layer "F.Cu") (at 127.814667 132.67618 -90)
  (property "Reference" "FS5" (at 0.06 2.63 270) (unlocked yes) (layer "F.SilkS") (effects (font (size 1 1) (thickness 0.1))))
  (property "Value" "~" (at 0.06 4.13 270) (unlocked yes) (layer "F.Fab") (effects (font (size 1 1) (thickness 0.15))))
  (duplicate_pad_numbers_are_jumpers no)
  (pad "" smd roundrect (at -0.75 0.01 180) (size 2 1) (layers "F.Mask" "F.Paste") (roundrect_rratio 0.2)
   (teardrops (best_length_ratio 0.5) (max_length 1) (best_width_ratio 1) (max_width 2) (curved_edges yes) (filter_ratio 0.9) (enabled yes)
    (allow_two_segments yes) (prefer_zone_connections yes)))
  (pad "" smd roundrect (at 0.75 0.01 180) (size 2 1) (layers "F.Mask" "F.Paste") (roundrect_rratio 0.2)
   (teardrops (best_length_ratio 0.5) (max_length 1) (best_width_ratio 1) (max_width 2) (curved_edges yes) (filter_ratio 0.9) (enabled yes)
    (allow_two_segments yes) (prefer_zone_connections yes)))
  (pad "1" smd roundrect (at 0.84 0 180) (size 2.82368 1.49099) (layers "F.Cu") (roundrect_rratio 0.25) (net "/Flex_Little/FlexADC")
   (teardrops (best_length_ratio 0.5) (max_length 1) (best_width_ratio 1) (max_width 2) (curved_edges yes) (filter_ratio 0.9) (enabled yes)
    (allow_two_segments yes) (prefer_zone_connections yes))
   (padstack (mode custom) (layer "B.Cu" (shape roundrect) (size 2.177876 1.183907) (roundrect_rratio 0.25) (zone_connect -1))))
  (pad "2" smd roundrect (at -0.87618 0.014667 180) (size 2.75 1.5) (layers "F.Cu") (roundrect_rratio 0.2) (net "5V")
   (teardrops (best_length_ratio 0.5) (max_length 1) (best_width_ratio 1) (max_width 2) (curved_edges yes) (filter_ratio 0.9) (enabled yes)
    (allow_two_segments yes) (prefer_zone_connections yes))))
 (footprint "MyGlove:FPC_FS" (layer "F.Cu") (at 109.76 114.2)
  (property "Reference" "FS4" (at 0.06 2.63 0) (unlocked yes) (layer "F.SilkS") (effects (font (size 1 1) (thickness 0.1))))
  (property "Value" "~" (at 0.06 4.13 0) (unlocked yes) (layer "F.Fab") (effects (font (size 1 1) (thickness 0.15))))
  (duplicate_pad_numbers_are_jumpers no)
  (pad "" smd roundrect (at -0.75 0.01 270) (size 2 1) (layers "F.Mask" "F.Paste") (roundrect_rratio 0.2)
   (teardrops (best_length_ratio 0.5) (max_length 1) (best_width_ratio 1) (max_width 2) (curved_edges yes) (filter_ratio 0.9) (enabled yes)
    (allow_two_segments yes) (prefer_zone_connections yes)))
  (pad "" smd roundrect (at 0.75 0.01 270) (size 2 1) (layers "F.Mask" "F.Paste") (roundrect_rratio 0.2)
   (teardrops (best_length_ratio 0.5) (max_length 1) (best_width_ratio 1) (max_width 2) (curved_edges yes) (filter_ratio 0.9) (enabled yes)
    (allow_two_segments yes) (prefer_zone_connections yes)))
  (pad "1" smd roundrect (at 0.84 0 270) (size 2.82368 1.49099) (layers "F.Cu") (roundrect_rratio 0.25) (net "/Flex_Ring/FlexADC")
   (teardrops (best_length_ratio 0.5) (max_length 1) (best_width_ratio 1) (max_width 2) (curved_edges yes) (filter_ratio 0.9) (enabled yes)
    (allow_two_segments yes) (prefer_zone_connections yes))
   (padstack (mode custom) (layer "B.Cu" (shape roundrect) (size 2.177876 1.183907) (roundrect_rratio 0.25) (zone_connect -1))))
  (pad "2" smd roundrect (at -0.87618 0.014667 270) (size 2.75 1.5) (layers "F.Cu") (roundrect_rratio 0.2) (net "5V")
   (teardrops (best_length_ratio 0.5) (max_length 1) (best_width_ratio 1) (max_width 2) (curved_edges yes) (filter_ratio 0.9) (enabled yes)
    (allow_two_segments yes) (prefer_zone_connections yes))))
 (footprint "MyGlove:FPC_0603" (layer "F.Cu") (at 89.3 141.5)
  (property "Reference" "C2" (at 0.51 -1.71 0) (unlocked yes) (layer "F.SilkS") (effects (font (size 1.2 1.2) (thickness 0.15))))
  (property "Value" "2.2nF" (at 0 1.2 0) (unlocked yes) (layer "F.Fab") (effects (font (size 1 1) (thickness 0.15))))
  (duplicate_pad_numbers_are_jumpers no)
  (pad "" smd roundrect (at -0.87 0.005971) (size 1.00047 0.948058) (layers "F.Mask" "F.Paste") (roundrect_rratio 0.2))
  (pad "" smd roundrect (at 0.85 0) (size 1.054536 0.970792) (layers "F.Mask" "F.Paste") (roundrect_rratio 0.2))
  (pad "1" smd roundrect (at -0.89 0.001664) (size 1.282964 1.211252) (layers "F.Cu") (roundrect_rratio 0.25) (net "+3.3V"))
  (pad "2" smd roundrect (at 0.86042 -0.015934) (size 1.289982 1.163733) (layers "F.Cu") (roundrect_rratio 0.25) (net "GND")))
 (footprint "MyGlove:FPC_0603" (layer "F.Cu") (at 89.2 133.4)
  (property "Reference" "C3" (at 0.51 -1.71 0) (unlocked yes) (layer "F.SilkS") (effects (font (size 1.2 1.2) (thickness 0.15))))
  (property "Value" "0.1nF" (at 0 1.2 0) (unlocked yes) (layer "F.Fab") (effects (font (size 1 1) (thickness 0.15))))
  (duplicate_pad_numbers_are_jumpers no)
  (pad "" smd roundrect (at -0.87 0.005971) (size 1.00047 0.948058) (layers "F.Mask" "F.Paste") (roundrect_rratio 0.2))
  (pad "" smd roundrect (at 0.85 0) (size 1.054536 0.970792) (layers "F.Mask" "F.Paste") (roundrect_rratio 0.2))
  (pad "1" smd roundrect (at -0.89 0.001664) (size 1.282964 1.211252) (layers "F.Cu") (roundrect_rratio 0.25) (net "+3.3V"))
  (pad "2" smd roundrect (at 0.86042 -0.015934) (size 1.289982 1.163733) (layers "F.Cu") (roundrect_rratio 0.25) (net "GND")))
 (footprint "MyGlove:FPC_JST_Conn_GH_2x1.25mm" (layer "F.Cu") (at 166.14 45.135 -90)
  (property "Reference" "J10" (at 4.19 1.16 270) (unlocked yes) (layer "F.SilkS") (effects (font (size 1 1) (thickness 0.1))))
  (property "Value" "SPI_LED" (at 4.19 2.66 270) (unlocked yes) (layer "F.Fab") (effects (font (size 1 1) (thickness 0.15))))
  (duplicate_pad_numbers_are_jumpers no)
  (pad "" smd roundrect (at 1.065 -2.46 270) (size 1 2.7) (layers "F.Mask" "F.Paste") (roundrect_rratio 0.25))
  (pad "" smd roundrect (at 2.915 -5.66 270) (size 0.6 1.7) (layers "F.Mask" "F.Paste") (roundrect_rratio 0.25))
  (pad "" smd roundrect (at 4.165 -5.66 270) (size 0.6 1.7) (layers "F.Mask" "F.Paste") (roundrect_rratio 0.25))
  (pad "" smd roundrect (at 6.015 -2.46 270) (size 1 2.7) (layers "F.Mask" "F.Paste") (roundrect_rratio 0.25))
  (pad "1" smd roundrect (at 2.788342 -5.567869 270) (size 1.129302 2.266628) (layers "F.Cu") (roundrect_rratio 0.25) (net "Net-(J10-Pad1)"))
  (pad "2" smd roundrect (at 4.303271 -5.565223 270) (size 1.113457 2.237746) (layers "F.Cu") (roundrect_rratio 0.25) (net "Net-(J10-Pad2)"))
  (pad "MP" smd roundrect (at 1.001135 -2.3257 270) (size 1.974193 3.465998) (layers "F.Cu") (roundrect_rratio 0.25))
  (pad "MP" smd roundrect (at 5.965717 -2.312819 270) (size 2.110214 3.455616) (layers "F.Cu") (roundrect_rratio 0.25)))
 (gr_poly
  (pts (xy 66.757031 195.041225) (xy 107.024648 195.193475) (xy 107.08287 187.394369) (xy 108.492513 179.845362) (xy 125.1 140.6)
   (xy 131.541065 136.913108) (xy 140.178734 139.126487) (xy 152.241065 133.113108) (xy 151.941065 126.013108) (xy 157.441065 121.613108)
   (xy 163.641065 122.513108) (xy 176.441065 114.313108) (xy 176.741065 109.113108) (xy 180.841065 105.413108) (xy 185.441065 108.313108)
   (xy 198.225552 100.106184) (xy 196.625552 85.906184) (xy 185.189232 83.22729) (xy 175.641065 90.913108) (xy 176.741065 96.713108)
   (xy 172.641065 99.413108) (xy 164.841065 96.513108) (xy 153.825552 104.406184) (xy 151.941065 111.513108) (xy 145.541065 115.713108)
   (xy 139.641065 111.813108) (xy 130.025552 116.806184) (xy 126.441065 125.613108) (xy 118.825552 127.806184) (xy 112.625552 125.806184)
   (xy 113.125552 119.306184) (xy 118.225552 116.406184) (xy 126.925552 114.806184) (xy 145.825552 97.506184) (xy 145.925552 86.706184)
   (xy 148.625552 83.606184) (xy 154.325552 85.906184) (xy 165.825552 73.706184) (xy 162.425552 66.506184) (xy 165.525552 63.306184)
   (xy 171.225552 66.006184) (xy 181.525552 53.806184) (xy 176.725552 42.306184) (xy 165.725552 38.706184) (xy 155.925552 50.106184)
   (xy 157.425552 52.206184) (xy 155.425552 55.806184) (xy 147.925552 54.006184) (xy 137.625552 68.906184) (xy 139.625552 74.006184)
   (xy 136.025552 78.306184) (xy 124.725552 78.106184) (xy 110.525552 99.606184) (xy 108.025552 106.706184) (xy 99.625552 110.806184)
   (xy 101.825552 101.906184) (xy 108.325552 98.206184) (xy 124.325552 71.406184) (xy 117.925552 61.806184) (xy 119.525552 57.906184)
   (xy 129.725552 59.806184) (xy 134.425552 48.706184) (xy 132.025552 37.506184) (xy 136.825552 31.106184) (xy 143.525552 29.706184)
   (xy 150.125552 18.806184) (xy 144.225552 8.006184) (xy 131.425552 8.206184) (xy 124.725552 18.306184) (xy 126.325552 23.406184)
   (xy 123.125552 28.806184) (xy 114.925552 28.406184) (xy 105.725552 45.606184) (xy 108.725552 51.306184) (xy 105.925552 57.006184)
   (xy 93.225552 59.306184) (xy 85.825552 84.506184) (xy 87.225552 93.206184) (xy 79.425552 102.306184) (xy 77.625552 91.606184)
   (xy 84.025552 85.106184) (xy 89.725552 60.406184) (xy 81.225552 54.206184) (xy 83.525552 46.906184) (xy 89.225552 45.306184)
   (xy 93.425552 28.806184) (xy 87.025552 25.406184) (xy 86.325552 16.506184) (xy 93.125552 13.406184) (xy 92.925552 -2.393816)
   (xy 79.725552 -10.793816) (xy 68.225552 -2.293816) (xy 68.025552 12.106184) (xy 72.825552 16.006184) (xy 73.225552 23.306184)
   (xy 64.825552 27.906184) (xy 63.225552 44.106184) (xy 69.425552 47.606184) (xy 68.425552 53.306184) (xy 61.125552 55.806184)
   (xy 55.225552 78.206184) (xy 63.625552 90.606184) (xy 64.325552 99.006184) (xy 54.125552 160.206184) (xy 54.125552 167.806184)
   (xy 41.125552 169.406184) (xy 32.925552 158.806184) (xy 21.425552 110.006184) (xy 37.625552 102.806184) (xy 37.625552 88.506184)
   (xy 18.025552 84.206184) (xy 18.625552 77.906184) (xy 39.625552 73.006184) (xy 40.725552 58.906184) (xy 22.425552 44.306184)
   (xy 11.625552 44.706184) (xy 5.225552 66.906184) (xy 7.225552 75.106184) (xy 6.825552 83.906184) (xy 2.425552 87.106184)
   (xy 0.625552 105.106184) (xy 8.025552 110.906184) (xy 12.625552 139.806184) (xy 20.425552 162.306184) (xy 31.925552 182.206184)
   (xy 35.625552 188.106184) (xy 41.025552 189.706184) (xy 64.525552 186.006184) (xy 66.825552 195.006184))
  (stroke (width 0.2) (type solid)) (fill no) (layer "Edge.Cuts"))
 (segment (start 89.804015 138.663379) (end 89.804015 141.127661) (width 0.3) (layer "F.Cu") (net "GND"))
 (segment (start 90.06042 133.384066) (end 90.06042 133.472084) (width 0.3) (layer "F.Cu") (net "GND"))
 (segment (start 93.413338 136.825002) (end 90.635 136.825002) (width 0.3) (layer "F.Cu") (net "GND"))
 (segment (start 89.804015 141.127661) (end 90.16042 141.484066) (width 0.3) (layer "F.Cu") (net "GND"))
 (segment (start 90.06042 133.472084) (end 93.498336 136.91) (width 0.3) (layer "F.Cu") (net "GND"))
 (segment (start 93.498336 136.91) (end 93.413338 136.825002) (width 0.3) (layer "F.Cu") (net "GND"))
 (segment (start 88.41 139.026968) (end 88.775002 138.661966) (width 0.3) (layer "F.Cu") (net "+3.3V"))
 (segment (start 90.073854 136.312407) (end 89.844457 136.541804) (width 0.3) (layer "F.Cu") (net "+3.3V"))
 (segment (start 88.41 141.501664) (end 88.41 139.026968) (width 0.3) (layer "F.Cu") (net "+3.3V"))
 (segment (start 88.31 133.401664) (end 90.073854 135.165518) (width 0.3) (layer "F.Cu") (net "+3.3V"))
 (segment (start 90.073854 135.165518) (end 90.073854 136.312407) (width 0.3) (layer "F.Cu") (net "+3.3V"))
 (segment (start 90.931963 138.66042) (end 90.636593 138.36505) (width 0.3) (layer "F.Cu") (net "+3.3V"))
 (segment (start 93.515934 138.66042) (end 90.931963 138.66042) (width 0.3) (layer "F.Cu") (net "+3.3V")))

